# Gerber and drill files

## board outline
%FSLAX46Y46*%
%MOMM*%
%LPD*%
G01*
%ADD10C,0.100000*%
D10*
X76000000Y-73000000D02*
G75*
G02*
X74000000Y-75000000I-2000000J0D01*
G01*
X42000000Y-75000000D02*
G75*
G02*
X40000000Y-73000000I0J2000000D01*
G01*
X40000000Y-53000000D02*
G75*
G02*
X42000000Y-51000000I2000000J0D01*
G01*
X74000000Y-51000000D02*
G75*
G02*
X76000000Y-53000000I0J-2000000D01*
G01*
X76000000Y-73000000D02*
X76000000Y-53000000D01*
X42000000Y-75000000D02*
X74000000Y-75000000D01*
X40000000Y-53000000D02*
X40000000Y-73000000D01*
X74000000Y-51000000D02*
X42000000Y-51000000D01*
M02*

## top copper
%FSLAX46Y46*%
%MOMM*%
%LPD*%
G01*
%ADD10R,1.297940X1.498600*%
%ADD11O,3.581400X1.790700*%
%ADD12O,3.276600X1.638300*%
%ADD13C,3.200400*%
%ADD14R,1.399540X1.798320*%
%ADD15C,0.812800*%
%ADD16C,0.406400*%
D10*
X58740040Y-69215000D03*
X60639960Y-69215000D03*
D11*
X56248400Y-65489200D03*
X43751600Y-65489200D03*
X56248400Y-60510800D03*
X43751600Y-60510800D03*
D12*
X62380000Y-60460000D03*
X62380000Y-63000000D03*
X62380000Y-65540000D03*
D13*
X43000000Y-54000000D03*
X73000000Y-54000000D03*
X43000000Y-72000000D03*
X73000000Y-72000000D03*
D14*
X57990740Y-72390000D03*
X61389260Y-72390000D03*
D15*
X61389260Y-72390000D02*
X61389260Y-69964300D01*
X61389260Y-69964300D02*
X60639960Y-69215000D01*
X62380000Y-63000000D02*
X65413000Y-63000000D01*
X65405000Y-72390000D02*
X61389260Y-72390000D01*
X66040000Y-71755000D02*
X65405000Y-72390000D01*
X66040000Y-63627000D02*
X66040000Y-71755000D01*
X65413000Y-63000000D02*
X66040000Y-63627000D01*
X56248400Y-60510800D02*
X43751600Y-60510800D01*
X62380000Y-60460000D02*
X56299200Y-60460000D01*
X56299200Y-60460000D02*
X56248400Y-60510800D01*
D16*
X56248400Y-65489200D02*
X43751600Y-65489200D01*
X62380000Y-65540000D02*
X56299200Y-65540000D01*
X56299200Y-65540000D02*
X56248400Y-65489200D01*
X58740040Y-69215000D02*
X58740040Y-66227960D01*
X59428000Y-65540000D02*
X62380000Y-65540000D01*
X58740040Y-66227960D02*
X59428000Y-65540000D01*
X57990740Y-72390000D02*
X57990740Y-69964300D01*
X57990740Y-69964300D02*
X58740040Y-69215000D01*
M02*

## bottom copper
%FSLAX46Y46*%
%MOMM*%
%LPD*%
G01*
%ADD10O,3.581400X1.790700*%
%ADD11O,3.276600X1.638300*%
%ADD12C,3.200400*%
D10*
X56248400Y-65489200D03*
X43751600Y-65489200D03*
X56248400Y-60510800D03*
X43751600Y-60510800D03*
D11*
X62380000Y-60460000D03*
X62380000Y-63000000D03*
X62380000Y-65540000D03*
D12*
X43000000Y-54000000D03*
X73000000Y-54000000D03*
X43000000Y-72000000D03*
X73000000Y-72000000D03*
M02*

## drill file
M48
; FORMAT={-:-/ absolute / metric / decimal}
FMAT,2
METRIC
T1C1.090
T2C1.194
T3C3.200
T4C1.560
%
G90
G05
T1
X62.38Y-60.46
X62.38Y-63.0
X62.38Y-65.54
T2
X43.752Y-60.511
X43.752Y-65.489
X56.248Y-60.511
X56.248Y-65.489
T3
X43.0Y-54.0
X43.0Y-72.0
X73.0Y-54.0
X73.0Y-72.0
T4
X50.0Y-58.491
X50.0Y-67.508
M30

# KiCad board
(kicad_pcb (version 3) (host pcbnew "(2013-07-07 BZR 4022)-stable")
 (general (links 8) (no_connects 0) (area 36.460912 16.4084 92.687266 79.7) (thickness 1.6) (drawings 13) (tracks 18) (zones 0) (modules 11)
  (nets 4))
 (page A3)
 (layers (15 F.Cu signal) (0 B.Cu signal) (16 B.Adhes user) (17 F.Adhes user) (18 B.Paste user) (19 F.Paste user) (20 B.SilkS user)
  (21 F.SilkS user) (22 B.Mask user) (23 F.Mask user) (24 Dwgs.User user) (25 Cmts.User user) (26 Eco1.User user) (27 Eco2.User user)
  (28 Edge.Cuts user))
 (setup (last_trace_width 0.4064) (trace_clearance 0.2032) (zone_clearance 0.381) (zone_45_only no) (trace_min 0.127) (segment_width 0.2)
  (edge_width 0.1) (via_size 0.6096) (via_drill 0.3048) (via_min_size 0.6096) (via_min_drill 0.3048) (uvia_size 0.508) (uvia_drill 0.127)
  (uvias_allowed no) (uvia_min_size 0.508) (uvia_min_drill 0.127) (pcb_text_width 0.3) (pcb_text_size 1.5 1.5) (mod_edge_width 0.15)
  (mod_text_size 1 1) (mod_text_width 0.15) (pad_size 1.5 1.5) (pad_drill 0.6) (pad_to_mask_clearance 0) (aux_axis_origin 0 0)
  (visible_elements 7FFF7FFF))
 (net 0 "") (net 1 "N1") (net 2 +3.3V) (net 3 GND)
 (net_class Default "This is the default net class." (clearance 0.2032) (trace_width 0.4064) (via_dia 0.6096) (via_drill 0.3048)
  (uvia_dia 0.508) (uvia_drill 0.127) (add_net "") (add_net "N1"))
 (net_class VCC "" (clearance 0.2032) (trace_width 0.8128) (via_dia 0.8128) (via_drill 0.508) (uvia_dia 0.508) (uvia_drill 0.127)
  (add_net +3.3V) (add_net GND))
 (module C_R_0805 (layer F.Cu) (at 59.69 69.215)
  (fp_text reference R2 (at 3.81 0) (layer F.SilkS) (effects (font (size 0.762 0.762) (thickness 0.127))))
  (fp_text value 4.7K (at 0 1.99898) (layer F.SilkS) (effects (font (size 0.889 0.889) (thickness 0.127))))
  (pad 1 smd rect (at -0.94996 0) (size 1.29794 1.4986) (layers F.Cu F.Paste F.SilkS F.Mask) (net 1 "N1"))
  (pad 2 smd rect (at 0.94996 0) (size 1.29794 1.4986) (layers F.Cu F.Paste F.SilkS F.Mask) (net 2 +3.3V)))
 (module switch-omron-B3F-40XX (layer F.Cu) (at 50 63 180)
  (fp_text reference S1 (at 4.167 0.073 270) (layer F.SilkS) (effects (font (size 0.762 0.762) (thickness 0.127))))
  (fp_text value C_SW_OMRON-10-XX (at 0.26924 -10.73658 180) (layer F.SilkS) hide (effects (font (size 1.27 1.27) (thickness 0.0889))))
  (pad "" np_thru_hole circle (at 0 4.5085 180) (size 1.55956 1.55956) (drill 1.55956) (layers *.Cu *.Paste *.SilkS *.Mask))
  (pad 1 thru_hole oval (at -6.2484 -2.4892 270) (size 1.7907 3.5814) (drill 1.193799) (layers *.Cu *.Adhes *.Paste *.SilkS *.Mask)
   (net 1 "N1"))
  (pad 2 thru_hole oval (at 6.2484 -2.4892 270) (size 1.7907 3.5814) (drill 1.193799) (layers *.Cu *.Adhes *.Paste *.SilkS *.Mask)
   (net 1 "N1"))
  (pad 3 thru_hole oval (at -6.2484 2.4892 270) (size 1.7907 3.5814) (drill 1.193799) (layers *.Cu *.Adhes *.Paste *.SilkS *.Mask)
   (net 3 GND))
  (pad 4 thru_hole oval (at 6.2484 2.4892 270) (size 1.7907 3.5814) (drill 1.193799) (layers *.Cu *.Adhes *.Paste *.SilkS *.Mask)
   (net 3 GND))
  (pad "" np_thru_hole circle (at 0 -4.5085 180) (size 1.55956 1.55956) (drill 1.55956) (layers *.Cu *.Paste *.SilkS *.Mask)))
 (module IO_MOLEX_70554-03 (layer F.Cu) (at 70 63 270)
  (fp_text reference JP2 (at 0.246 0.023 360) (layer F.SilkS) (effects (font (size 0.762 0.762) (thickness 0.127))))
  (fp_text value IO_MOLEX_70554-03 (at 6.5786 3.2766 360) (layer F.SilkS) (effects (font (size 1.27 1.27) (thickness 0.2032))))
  (pad 1 thru_hole oval (at -2.54 7.62 270) (size 1.6383 3.2766) (drill 1.08966) (layers *.Cu *.Adhes *.Paste *.SilkS *.Mask) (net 3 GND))
  (pad 2 thru_hole oval (at 0 7.62 270) (size 1.6383 3.2766) (drill 1.08966) (layers *.Cu *.Adhes *.Paste *.SilkS *.Mask) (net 2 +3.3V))
  (pad 3 thru_hole oval (at 2.54 7.62 270) (size 1.6383 3.2766) (drill 1.08966) (layers *.Cu *.Adhes *.Paste *.SilkS *.Mask) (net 1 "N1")))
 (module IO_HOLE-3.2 (layer F.Cu) (at 43 54)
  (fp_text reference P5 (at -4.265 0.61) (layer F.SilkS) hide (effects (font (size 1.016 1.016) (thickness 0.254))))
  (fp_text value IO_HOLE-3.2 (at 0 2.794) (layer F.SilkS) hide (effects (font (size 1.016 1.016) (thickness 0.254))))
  (pad "" thru_hole circle (at 0 0) (size 3.2004 3.2004) (drill 3.2004) (layers *.Cu *.Paste *.SilkS *.Mask)))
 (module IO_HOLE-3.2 (layer F.Cu) (at 73 54)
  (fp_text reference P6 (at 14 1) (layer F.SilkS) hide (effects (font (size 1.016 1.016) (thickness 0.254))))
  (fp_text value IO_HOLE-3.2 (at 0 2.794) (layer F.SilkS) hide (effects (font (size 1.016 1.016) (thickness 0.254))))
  (pad "" thru_hole circle (at 0 0) (size 3.2004 3.2004) (drill 3.2004) (layers *.Cu *.Paste *.SilkS *.Mask)))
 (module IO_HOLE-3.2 (layer F.Cu) (at 43 72)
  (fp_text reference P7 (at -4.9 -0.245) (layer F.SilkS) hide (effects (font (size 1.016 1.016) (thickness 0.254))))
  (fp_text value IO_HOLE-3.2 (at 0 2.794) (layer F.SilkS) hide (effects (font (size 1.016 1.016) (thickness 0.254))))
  (pad "" thru_hole circle (at 0 0) (size 3.2004 3.2004) (drill 3.2004) (layers *.Cu *.Paste *.SilkS *.Mask)))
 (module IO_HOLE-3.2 (layer F.Cu) (at 73 72)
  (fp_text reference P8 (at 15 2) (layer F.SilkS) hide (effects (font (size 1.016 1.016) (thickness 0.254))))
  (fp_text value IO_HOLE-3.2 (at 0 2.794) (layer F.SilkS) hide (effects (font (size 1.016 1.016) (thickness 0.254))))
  (pad "" thru_hole circle (at 0 0) (size 3.2004 3.2004) (drill 3.2004) (layers *.Cu *.Paste *.SilkS *.Mask)))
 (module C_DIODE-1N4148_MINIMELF (layer F.Cu) (at 59.69 72.39 180)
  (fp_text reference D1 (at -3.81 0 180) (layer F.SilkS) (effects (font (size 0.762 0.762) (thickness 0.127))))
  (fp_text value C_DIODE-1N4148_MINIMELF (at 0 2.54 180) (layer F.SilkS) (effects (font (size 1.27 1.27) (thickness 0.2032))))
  (pad 1 smd rect (at 1.69926 0 180) (size 1.39954 1.79832) (layers F.Cu F.Paste F.Mask) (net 1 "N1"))
  (pad 2 smd rect (at -1.69926 0 180) (size 1.39954 1.79832) (layers F.Cu F.Paste F.Mask) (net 2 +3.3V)))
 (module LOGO (layer F.Cu) (at 67.945 55.245)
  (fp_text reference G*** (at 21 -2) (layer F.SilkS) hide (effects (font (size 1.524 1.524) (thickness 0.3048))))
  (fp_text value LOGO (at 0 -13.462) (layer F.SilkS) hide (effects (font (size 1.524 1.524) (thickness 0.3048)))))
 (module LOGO (layer F.Cu) (at 59.055 54.991)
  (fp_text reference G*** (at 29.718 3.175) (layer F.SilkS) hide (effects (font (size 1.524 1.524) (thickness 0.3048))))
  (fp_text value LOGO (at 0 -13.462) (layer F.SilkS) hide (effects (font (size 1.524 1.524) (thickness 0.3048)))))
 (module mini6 (layer B.Cu) (at 56 65)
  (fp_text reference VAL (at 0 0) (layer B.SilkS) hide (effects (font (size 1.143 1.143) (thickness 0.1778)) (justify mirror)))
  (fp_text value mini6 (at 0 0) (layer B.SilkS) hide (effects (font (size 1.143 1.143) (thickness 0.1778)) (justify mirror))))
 (gr_arc (start 74 73) (end 76 73) (angle 90) (layer Edge.Cuts) (width 0.1))
 (gr_arc (start 42 73) (end 42 75) (angle 90) (layer Edge.Cuts) (width 0.1))
 (gr_arc (start 42 53) (end 40 53) (angle 90) (layer Edge.Cuts) (width 0.1))
 (gr_arc (start 74 53) (end 74 51) (angle 90) (layer Edge.Cuts) (width 0.1))
 (gr_line (start 76 73) (end 76 53) (angle 90) (layer Edge.Cuts) (width 0.1))
 (gr_line (start 42 75) (end 74 75) (angle 90) (layer Edge.Cuts) (width 0.1))
 (gr_line (start 40 53) (end 40 73) (angle 90) (layer Edge.Cuts) (width 0.1))
 (gr_line (start 74 51) (end 42 51) (angle 90) (layer Edge.Cuts) (width 0.1))
 (segment (start 61.38926 72.39) (end 61.38926 69.9643) (width 0.8128) (layer F.Cu) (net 2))
 (segment (start 61.38926 69.9643) (end 60.63996 69.215) (width 0.8128) (layer F.Cu) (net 2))
 (segment (start 62.38 63) (end 65.413 63) (width 0.8128) (layer F.Cu) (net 2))
 (segment (start 65.405 72.39) (end 61.38926 72.39) (width 0.8128) (layer F.Cu) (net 2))
 (segment (start 66.04 71.755) (end 65.405 72.39) (width 0.8128) (layer F.Cu) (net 2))
 (segment (start 66.04 63.627) (end 66.04 71.755) (width 0.8128) (layer F.Cu) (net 2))
 (segment (start 65.413 63) (end 66.04 63.627) (width 0.8128) (layer F.Cu) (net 2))
 (segment (start 56.2484 60.5108) (end 43.7516 60.5108) (width 0.8128) (layer F.Cu) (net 3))
 (segment (start 62.38 60.46) (end 56.2992 60.46) (width 0.8128) (layer F.Cu) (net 3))
 (segment (start 56.2992 60.46) (end 56.2484 60.5108) (width 0.8128) (layer F.Cu) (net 3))
 (segment (start 56.2484 65.4892) (end 43.7516 65.4892) (width 0.4064) (layer F.Cu) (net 1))
 (segment (start 62.38 65.54) (end 56.2992 65.54) (width 0.4064) (layer F.Cu) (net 1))
 (segment (start 56.2992 65.54) (end 56.2484 65.4892) (width 0.4064) (layer F.Cu) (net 1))
 (segment (start 58.74004 69.215) (end 58.74004 66.22796) (width 0.4064) (layer F.Cu) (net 1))
 (segment (start 59.428 65.54) (end 62.38 65.54) (width 0.4064) (layer F.Cu) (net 1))
 (segment (start 58.74004 66.22796) (end 59.428 65.54) (width 0.4064) (layer F.Cu) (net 1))
 (segment (start 57.99074 72.39) (end 57.99074 69.9643) (width 0.4064) (layer F.Cu) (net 1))
 (segment (start 57.99074 69.9643) (end 58.74004 69.215) (width 0.4064) (layer F.Cu) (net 1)))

